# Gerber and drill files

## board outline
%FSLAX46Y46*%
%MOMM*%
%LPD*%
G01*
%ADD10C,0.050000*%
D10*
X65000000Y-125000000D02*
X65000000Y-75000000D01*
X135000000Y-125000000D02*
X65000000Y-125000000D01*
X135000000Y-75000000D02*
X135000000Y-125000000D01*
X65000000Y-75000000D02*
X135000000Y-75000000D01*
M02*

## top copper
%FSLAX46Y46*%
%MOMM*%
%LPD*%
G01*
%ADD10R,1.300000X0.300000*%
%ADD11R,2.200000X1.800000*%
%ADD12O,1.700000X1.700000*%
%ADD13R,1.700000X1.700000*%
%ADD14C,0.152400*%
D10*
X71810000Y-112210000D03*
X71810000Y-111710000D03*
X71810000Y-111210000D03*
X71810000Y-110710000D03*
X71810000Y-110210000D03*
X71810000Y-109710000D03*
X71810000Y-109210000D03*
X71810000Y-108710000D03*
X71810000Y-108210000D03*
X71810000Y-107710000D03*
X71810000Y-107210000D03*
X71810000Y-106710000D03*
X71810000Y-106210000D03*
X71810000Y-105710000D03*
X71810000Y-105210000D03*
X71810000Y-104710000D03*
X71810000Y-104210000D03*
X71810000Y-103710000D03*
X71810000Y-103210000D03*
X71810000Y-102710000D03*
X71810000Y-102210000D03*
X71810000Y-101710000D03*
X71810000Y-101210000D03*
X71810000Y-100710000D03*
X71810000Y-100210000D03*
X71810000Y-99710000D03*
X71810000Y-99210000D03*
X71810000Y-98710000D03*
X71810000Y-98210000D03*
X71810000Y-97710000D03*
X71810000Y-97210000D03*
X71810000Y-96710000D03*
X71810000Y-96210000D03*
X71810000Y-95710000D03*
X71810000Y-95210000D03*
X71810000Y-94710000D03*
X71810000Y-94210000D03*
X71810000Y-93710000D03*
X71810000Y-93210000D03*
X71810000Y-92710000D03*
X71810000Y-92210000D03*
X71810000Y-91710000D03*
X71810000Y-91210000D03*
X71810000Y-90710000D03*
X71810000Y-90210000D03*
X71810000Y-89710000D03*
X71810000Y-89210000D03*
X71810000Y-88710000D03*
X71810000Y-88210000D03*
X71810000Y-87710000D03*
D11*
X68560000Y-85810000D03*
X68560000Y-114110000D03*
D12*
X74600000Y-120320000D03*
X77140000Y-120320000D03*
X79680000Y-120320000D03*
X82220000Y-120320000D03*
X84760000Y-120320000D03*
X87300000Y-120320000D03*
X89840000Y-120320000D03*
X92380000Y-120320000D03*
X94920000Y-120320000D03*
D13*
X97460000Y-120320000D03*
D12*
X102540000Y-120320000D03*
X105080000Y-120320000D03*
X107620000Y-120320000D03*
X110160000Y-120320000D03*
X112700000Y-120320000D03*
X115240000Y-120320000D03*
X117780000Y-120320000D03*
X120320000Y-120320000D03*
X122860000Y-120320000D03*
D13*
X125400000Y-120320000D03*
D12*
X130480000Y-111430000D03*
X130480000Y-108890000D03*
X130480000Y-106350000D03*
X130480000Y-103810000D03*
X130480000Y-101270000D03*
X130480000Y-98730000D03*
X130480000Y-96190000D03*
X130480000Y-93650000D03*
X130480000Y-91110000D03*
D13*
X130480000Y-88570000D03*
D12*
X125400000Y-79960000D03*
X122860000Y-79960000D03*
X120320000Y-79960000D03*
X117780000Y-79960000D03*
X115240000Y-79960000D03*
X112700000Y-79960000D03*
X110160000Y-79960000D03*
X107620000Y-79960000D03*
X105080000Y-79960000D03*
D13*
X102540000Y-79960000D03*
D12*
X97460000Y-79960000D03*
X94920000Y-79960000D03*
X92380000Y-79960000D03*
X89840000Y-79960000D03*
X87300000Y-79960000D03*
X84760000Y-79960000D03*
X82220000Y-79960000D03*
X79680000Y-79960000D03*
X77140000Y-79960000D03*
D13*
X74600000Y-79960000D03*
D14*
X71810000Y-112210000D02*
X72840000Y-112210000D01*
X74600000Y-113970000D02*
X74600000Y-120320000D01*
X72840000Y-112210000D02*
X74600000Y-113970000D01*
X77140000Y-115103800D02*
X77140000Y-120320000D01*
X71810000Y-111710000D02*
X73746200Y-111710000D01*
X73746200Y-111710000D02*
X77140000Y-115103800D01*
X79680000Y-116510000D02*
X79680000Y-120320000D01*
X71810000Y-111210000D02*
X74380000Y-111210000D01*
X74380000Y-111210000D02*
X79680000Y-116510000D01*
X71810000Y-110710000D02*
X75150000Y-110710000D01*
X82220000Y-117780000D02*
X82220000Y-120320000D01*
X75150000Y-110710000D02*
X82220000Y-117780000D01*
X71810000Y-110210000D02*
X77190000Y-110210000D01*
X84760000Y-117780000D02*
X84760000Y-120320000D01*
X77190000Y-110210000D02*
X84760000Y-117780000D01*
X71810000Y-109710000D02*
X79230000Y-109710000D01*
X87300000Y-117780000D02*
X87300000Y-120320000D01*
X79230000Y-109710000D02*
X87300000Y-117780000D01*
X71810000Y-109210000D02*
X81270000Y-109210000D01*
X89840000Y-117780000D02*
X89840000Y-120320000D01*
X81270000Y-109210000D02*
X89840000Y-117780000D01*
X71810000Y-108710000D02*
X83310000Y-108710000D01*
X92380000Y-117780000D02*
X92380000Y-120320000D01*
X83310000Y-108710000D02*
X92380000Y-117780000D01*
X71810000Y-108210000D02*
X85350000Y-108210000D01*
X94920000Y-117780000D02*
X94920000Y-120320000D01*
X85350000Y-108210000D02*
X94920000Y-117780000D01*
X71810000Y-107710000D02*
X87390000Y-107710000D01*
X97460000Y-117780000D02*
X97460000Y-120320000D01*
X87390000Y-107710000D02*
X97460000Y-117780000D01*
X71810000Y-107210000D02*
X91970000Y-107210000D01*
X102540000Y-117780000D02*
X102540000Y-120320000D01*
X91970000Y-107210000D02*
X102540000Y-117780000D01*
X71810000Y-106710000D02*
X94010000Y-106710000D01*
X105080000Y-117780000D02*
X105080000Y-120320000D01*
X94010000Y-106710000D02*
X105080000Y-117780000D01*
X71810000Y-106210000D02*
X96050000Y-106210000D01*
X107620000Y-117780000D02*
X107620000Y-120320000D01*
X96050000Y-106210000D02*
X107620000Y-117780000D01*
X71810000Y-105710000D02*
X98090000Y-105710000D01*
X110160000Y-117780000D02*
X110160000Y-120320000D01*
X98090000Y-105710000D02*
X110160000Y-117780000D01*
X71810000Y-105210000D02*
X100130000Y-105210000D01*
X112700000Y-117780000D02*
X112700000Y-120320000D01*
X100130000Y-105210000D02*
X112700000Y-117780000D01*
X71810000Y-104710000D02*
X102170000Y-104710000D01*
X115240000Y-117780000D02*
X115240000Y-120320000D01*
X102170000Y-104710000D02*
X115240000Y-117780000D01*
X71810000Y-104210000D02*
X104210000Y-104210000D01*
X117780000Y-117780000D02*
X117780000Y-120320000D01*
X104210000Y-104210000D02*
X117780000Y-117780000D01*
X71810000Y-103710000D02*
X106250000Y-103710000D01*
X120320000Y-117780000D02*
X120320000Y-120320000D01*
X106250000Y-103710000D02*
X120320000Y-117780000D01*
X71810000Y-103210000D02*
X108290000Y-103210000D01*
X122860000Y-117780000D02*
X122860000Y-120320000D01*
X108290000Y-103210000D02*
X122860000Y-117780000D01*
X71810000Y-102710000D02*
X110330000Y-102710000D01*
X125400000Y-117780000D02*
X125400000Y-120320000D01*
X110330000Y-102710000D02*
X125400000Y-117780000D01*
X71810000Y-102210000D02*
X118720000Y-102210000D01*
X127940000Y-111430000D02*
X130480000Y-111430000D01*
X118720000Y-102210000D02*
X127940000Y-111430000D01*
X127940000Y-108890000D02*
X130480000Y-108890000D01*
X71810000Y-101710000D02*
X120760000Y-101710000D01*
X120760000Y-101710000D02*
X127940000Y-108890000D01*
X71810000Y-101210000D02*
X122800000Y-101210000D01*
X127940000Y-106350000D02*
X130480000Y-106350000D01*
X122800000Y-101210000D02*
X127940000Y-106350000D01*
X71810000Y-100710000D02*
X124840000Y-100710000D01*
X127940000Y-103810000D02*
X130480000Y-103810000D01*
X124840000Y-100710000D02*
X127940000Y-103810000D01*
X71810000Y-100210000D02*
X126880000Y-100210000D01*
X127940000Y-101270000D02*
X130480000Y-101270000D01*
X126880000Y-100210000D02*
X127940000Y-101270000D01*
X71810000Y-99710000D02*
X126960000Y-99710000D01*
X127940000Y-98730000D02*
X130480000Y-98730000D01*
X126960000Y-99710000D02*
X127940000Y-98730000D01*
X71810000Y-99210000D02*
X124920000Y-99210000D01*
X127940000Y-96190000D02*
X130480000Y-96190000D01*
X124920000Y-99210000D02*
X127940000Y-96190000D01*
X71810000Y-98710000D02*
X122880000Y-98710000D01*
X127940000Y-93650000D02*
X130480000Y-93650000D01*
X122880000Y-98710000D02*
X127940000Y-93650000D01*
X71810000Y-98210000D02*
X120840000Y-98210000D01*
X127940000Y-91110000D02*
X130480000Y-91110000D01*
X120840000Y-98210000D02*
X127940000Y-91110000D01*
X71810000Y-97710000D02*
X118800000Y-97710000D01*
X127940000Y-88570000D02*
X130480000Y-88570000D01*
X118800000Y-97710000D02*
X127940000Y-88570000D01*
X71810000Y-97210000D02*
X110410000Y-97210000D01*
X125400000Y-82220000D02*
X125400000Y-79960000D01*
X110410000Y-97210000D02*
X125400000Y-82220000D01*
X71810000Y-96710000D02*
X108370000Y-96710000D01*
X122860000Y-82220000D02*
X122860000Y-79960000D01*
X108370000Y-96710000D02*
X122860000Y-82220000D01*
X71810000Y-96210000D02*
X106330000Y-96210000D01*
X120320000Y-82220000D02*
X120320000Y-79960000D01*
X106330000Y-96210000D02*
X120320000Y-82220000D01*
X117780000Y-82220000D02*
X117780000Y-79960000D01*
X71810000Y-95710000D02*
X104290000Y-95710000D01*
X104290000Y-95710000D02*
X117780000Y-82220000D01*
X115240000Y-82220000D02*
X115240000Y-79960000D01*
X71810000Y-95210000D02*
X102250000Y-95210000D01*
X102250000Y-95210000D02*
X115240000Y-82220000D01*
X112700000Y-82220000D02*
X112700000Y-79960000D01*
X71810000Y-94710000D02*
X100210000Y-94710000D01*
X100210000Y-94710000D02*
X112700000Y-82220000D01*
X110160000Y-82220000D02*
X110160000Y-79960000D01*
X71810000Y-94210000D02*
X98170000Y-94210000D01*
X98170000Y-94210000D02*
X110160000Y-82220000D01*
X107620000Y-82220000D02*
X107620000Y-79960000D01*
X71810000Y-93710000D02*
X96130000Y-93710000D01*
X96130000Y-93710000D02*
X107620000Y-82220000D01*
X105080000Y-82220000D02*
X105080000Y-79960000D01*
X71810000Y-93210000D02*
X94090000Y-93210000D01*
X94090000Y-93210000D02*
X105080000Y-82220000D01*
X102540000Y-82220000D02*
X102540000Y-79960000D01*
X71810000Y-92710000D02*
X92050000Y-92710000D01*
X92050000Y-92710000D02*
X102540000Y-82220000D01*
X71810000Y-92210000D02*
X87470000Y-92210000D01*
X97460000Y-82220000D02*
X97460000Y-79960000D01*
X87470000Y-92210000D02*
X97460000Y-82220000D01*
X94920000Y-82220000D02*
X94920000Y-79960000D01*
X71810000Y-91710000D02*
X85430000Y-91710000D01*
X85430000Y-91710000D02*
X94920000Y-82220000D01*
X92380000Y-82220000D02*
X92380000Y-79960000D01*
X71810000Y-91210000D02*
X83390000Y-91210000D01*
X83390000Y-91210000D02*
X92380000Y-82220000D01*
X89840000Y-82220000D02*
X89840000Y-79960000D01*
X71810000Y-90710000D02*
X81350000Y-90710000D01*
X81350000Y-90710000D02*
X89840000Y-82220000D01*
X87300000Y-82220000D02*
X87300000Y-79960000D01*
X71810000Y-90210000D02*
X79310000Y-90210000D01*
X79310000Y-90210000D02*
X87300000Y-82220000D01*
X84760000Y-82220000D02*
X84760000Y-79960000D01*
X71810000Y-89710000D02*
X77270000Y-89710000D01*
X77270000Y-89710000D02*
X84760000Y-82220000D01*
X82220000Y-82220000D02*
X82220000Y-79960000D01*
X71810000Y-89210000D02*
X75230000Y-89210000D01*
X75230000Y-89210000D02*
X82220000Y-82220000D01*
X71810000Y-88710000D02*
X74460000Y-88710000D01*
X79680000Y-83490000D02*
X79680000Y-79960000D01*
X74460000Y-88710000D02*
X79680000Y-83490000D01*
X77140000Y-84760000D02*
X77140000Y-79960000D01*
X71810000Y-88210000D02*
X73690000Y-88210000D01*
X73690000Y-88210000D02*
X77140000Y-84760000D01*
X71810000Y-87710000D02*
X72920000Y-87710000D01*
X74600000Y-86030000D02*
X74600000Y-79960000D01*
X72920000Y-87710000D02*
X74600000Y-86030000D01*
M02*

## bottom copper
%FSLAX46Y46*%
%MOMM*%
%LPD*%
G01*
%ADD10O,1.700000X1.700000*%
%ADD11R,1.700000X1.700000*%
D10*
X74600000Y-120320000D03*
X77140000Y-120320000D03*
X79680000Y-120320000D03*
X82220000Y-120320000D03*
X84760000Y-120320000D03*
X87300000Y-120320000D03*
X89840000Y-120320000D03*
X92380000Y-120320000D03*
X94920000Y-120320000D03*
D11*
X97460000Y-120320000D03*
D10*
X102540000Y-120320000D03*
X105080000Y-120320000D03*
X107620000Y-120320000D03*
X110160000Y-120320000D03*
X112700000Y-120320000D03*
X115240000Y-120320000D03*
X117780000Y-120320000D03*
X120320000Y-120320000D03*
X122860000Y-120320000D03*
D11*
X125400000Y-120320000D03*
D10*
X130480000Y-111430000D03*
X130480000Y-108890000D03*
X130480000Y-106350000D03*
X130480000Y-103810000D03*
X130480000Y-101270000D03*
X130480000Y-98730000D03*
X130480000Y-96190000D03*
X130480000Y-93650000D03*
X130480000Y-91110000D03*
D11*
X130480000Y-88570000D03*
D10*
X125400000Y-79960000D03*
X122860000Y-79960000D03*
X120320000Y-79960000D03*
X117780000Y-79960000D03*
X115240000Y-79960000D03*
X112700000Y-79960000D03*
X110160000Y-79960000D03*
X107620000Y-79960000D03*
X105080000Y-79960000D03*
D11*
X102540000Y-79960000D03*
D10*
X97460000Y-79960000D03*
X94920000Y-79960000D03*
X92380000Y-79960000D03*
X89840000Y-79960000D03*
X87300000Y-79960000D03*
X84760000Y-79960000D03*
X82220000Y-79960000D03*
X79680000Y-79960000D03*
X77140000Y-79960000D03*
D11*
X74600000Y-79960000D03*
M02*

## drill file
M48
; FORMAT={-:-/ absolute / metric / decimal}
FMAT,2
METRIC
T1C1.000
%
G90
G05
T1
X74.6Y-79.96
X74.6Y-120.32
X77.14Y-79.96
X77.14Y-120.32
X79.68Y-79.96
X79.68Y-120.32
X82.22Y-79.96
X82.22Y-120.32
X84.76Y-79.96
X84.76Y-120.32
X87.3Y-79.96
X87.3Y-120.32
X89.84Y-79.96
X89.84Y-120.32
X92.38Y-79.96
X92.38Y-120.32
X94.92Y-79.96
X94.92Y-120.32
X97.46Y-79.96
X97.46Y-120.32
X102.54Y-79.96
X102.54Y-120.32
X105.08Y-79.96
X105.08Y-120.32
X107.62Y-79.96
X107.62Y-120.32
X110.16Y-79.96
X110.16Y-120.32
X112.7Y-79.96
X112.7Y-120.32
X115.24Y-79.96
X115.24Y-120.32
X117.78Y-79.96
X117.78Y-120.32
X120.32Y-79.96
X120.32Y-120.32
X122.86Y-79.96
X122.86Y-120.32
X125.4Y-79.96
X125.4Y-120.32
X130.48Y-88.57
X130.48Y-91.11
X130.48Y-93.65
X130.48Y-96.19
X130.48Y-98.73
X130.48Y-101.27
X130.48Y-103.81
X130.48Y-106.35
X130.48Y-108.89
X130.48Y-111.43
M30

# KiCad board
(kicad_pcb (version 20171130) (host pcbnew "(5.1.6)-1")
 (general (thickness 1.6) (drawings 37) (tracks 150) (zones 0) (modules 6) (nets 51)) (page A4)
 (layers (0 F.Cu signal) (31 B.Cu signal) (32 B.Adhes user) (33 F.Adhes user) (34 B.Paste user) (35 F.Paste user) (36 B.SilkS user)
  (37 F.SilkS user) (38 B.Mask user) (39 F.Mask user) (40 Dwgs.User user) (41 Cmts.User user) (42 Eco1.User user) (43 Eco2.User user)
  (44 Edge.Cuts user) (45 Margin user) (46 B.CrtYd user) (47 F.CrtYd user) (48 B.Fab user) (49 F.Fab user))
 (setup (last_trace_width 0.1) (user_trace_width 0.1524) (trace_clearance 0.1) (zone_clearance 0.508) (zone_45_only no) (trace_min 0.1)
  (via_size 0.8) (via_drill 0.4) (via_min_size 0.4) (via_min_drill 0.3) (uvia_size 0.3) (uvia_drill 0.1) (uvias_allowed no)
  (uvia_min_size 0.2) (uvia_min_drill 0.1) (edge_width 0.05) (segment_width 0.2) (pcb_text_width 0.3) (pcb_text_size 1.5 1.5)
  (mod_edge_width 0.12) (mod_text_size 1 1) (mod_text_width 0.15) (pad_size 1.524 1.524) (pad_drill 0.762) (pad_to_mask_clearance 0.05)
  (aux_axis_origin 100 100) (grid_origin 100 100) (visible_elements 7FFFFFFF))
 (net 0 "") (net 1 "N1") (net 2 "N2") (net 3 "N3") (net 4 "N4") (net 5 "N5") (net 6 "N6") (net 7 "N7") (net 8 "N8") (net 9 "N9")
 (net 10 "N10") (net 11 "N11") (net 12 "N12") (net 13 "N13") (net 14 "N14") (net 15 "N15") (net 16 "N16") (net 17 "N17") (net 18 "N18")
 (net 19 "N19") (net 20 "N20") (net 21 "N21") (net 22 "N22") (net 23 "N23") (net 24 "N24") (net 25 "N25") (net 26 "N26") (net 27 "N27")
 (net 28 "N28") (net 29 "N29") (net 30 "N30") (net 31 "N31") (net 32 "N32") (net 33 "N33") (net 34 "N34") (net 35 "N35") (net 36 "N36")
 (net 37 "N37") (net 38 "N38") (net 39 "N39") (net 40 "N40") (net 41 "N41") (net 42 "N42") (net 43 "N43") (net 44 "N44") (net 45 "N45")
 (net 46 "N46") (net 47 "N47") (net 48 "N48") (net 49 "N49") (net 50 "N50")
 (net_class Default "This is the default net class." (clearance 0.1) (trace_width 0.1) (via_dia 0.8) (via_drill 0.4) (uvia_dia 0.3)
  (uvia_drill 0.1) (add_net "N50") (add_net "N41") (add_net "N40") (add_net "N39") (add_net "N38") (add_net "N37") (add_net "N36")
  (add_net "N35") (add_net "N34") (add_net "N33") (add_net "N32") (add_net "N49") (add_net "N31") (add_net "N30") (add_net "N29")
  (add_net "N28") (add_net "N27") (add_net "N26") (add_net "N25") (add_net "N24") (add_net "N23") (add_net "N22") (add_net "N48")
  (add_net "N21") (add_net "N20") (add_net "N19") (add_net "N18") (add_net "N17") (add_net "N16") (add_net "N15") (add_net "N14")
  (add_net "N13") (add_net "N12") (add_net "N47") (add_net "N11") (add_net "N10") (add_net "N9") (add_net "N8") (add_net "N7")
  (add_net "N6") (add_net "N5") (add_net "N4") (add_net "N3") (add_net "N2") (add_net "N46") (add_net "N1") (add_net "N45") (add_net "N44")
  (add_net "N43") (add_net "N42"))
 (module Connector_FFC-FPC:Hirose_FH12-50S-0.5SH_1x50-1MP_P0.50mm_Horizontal (layer F.Cu) (at 69.96 99.96 270)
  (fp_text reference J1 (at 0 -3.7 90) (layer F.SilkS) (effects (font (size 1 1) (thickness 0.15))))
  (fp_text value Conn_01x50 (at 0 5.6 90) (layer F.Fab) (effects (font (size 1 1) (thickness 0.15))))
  (pad 50 smd rect (at 12.25 -1.85 270) (size 0.3 1.3) (layers F.Cu F.Paste F.Mask) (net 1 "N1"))
  (pad 49 smd rect (at 11.75 -1.85 270) (size 0.3 1.3) (layers F.Cu F.Paste F.Mask) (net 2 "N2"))
  (pad 48 smd rect (at 11.25 -1.85 270) (size 0.3 1.3) (layers F.Cu F.Paste F.Mask) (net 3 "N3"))
  (pad 47 smd rect (at 10.75 -1.85 270) (size 0.3 1.3) (layers F.Cu F.Paste F.Mask) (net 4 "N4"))
  (pad 46 smd rect (at 10.25 -1.85 270) (size 0.3 1.3) (layers F.Cu F.Paste F.Mask) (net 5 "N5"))
  (pad 45 smd rect (at 9.75 -1.85 270) (size 0.3 1.3) (layers F.Cu F.Paste F.Mask) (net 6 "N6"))
  (pad 44 smd rect (at 9.25 -1.85 270) (size 0.3 1.3) (layers F.Cu F.Paste F.Mask) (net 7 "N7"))
  (pad 43 smd rect (at 8.75 -1.85 270) (size 0.3 1.3) (layers F.Cu F.Paste F.Mask) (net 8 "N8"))
  (pad 42 smd rect (at 8.25 -1.85 270) (size 0.3 1.3) (layers F.Cu F.Paste F.Mask) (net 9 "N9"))
  (pad 41 smd rect (at 7.75 -1.85 270) (size 0.3 1.3) (layers F.Cu F.Paste F.Mask) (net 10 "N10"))
  (pad 40 smd rect (at 7.25 -1.85 270) (size 0.3 1.3) (layers F.Cu F.Paste F.Mask) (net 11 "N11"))
  (pad 39 smd rect (at 6.75 -1.85 270) (size 0.3 1.3) (layers F.Cu F.Paste F.Mask) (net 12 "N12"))
  (pad 38 smd rect (at 6.25 -1.85 270) (size 0.3 1.3) (layers F.Cu F.Paste F.Mask) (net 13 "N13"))
  (pad 37 smd rect (at 5.75 -1.85 270) (size 0.3 1.3) (layers F.Cu F.Paste F.Mask) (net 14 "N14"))
  (pad 36 smd rect (at 5.25 -1.85 270) (size 0.3 1.3) (layers F.Cu F.Paste F.Mask) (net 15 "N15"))
  (pad 35 smd rect (at 4.75 -1.85 270) (size 0.3 1.3) (layers F.Cu F.Paste F.Mask) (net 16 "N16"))
  (pad 34 smd rect (at 4.25 -1.85 270) (size 0.3 1.3) (layers F.Cu F.Paste F.Mask) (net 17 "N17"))
  (pad 33 smd rect (at 3.75 -1.85 270) (size 0.3 1.3) (layers F.Cu F.Paste F.Mask) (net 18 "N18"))
  (pad 32 smd rect (at 3.25 -1.85 270) (size 0.3 1.3) (layers F.Cu F.Paste F.Mask) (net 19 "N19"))
  (pad 31 smd rect (at 2.75 -1.85 270) (size 0.3 1.3) (layers F.Cu F.Paste F.Mask) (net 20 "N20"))
  (pad 30 smd rect (at 2.25 -1.85 270) (size 0.3 1.3) (layers F.Cu F.Paste F.Mask) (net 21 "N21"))
  (pad 29 smd rect (at 1.75 -1.85 270) (size 0.3 1.3) (layers F.Cu F.Paste F.Mask) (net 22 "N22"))
  (pad 28 smd rect (at 1.25 -1.85 270) (size 0.3 1.3) (layers F.Cu F.Paste F.Mask) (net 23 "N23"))
  (pad 27 smd rect (at 0.75 -1.85 270) (size 0.3 1.3) (layers F.Cu F.Paste F.Mask) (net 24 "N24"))
  (pad 26 smd rect (at 0.25 -1.85 270) (size 0.3 1.3) (layers F.Cu F.Paste F.Mask) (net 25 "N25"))
  (pad 25 smd rect (at -0.25 -1.85 270) (size 0.3 1.3) (layers F.Cu F.Paste F.Mask) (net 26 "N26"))
  (pad 24 smd rect (at -0.75 -1.85 270) (size 0.3 1.3) (layers F.Cu F.Paste F.Mask) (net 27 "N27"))
  (pad 23 smd rect (at -1.25 -1.85 270) (size 0.3 1.3) (layers F.Cu F.Paste F.Mask) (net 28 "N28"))
  (pad 22 smd rect (at -1.75 -1.85 270) (size 0.3 1.3) (layers F.Cu F.Paste F.Mask) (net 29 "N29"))
  (pad 21 smd rect (at -2.25 -1.85 270) (size 0.3 1.3) (layers F.Cu F.Paste F.Mask) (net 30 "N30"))
  (pad 20 smd rect (at -2.75 -1.85 270) (size 0.3 1.3) (layers F.Cu F.Paste F.Mask) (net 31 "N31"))
  (pad 19 smd rect (at -3.25 -1.85 270) (size 0.3 1.3) (layers F.Cu F.Paste F.Mask) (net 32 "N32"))
  (pad 18 smd rect (at -3.75 -1.85 270) (size 0.3 1.3) (layers F.Cu F.Paste F.Mask) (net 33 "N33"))
  (pad 17 smd rect (at -4.25 -1.85 270) (size 0.3 1.3) (layers F.Cu F.Paste F.Mask) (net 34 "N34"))
  (pad 16 smd rect (at -4.75 -1.85 270) (size 0.3 1.3) (layers F.Cu F.Paste F.Mask) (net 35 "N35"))
  (pad 15 smd rect (at -5.25 -1.85 270) (size 0.3 1.3) (layers F.Cu F.Paste F.Mask) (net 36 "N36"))
  (pad 14 smd rect (at -5.75 -1.85 270) (size 0.3 1.3) (layers F.Cu F.Paste F.Mask) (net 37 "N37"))
  (pad 13 smd rect (at -6.25 -1.85 270) (size 0.3 1.3) (layers F.Cu F.Paste F.Mask) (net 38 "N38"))
  (pad 12 smd rect (at -6.75 -1.85 270) (size 0.3 1.3) (layers F.Cu F.Paste F.Mask) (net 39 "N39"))
  (pad 11 smd rect (at -7.25 -1.85 270) (size 0.3 1.3) (layers F.Cu F.Paste F.Mask) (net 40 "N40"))
  (pad 10 smd rect (at -7.75 -1.85 270) (size 0.3 1.3) (layers F.Cu F.Paste F.Mask) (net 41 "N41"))
  (pad 9 smd rect (at -8.25 -1.85 270) (size 0.3 1.3) (layers F.Cu F.Paste F.Mask) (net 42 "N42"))
  (pad 8 smd rect (at -8.75 -1.85 270) (size 0.3 1.3) (layers F.Cu F.Paste F.Mask) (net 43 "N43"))
  (pad 7 smd rect (at -9.25 -1.85 270) (size 0.3 1.3) (layers F.Cu F.Paste F.Mask) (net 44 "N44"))
  (pad 6 smd rect (at -9.75 -1.85 270) (size 0.3 1.3) (layers F.Cu F.Paste F.Mask) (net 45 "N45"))
  (pad 5 smd rect (at -10.25 -1.85 270) (size 0.3 1.3) (layers F.Cu F.Paste F.Mask) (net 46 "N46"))
  (pad 4 smd rect (at -10.75 -1.85 270) (size 0.3 1.3) (layers F.Cu F.Paste F.Mask) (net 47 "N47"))
  (pad 3 smd rect (at -11.25 -1.85 270) (size 0.3 1.3) (layers F.Cu F.Paste F.Mask) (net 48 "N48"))
  (pad 2 smd rect (at -11.75 -1.85 270) (size 0.3 1.3) (layers F.Cu F.Paste F.Mask) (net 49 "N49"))
  (pad 1 smd rect (at -12.25 -1.85 270) (size 0.3 1.3) (layers F.Cu F.Paste F.Mask) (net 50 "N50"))
  (pad MP smd rect (at -14.15 1.4 270) (size 1.8 2.2) (layers F.Cu F.Paste F.Mask))
  (pad MP smd rect (at 14.15 1.4 270) (size 1.8 2.2) (layers F.Cu F.Paste F.Mask)))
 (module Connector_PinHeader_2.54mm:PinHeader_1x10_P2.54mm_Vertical (layer F.Cu) (at 97.46 120.32 270)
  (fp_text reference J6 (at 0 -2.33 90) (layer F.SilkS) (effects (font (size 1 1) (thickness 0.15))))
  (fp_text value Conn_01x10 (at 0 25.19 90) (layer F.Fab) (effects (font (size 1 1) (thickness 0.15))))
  (pad 10 thru_hole oval (at 0 22.86 270) (size 1.7 1.7) (drill 1) (layers *.Cu *.Mask) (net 1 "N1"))
  (pad 9 thru_hole oval (at 0 20.32 270) (size 1.7 1.7) (drill 1) (layers *.Cu *.Mask) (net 2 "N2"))
  (pad 8 thru_hole oval (at 0 17.78 270) (size 1.7 1.7) (drill 1) (layers *.Cu *.Mask) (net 3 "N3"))
  (pad 7 thru_hole oval (at 0 15.24 270) (size 1.7 1.7) (drill 1) (layers *.Cu *.Mask) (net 4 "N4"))
  (pad 6 thru_hole oval (at 0 12.7 270) (size 1.7 1.7) (drill 1) (layers *.Cu *.Mask) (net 5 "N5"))
  (pad 5 thru_hole oval (at 0 10.16 270) (size 1.7 1.7) (drill 1) (layers *.Cu *.Mask) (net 6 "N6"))
  (pad 4 thru_hole oval (at 0 7.62 270) (size 1.7 1.7) (drill 1) (layers *.Cu *.Mask) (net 7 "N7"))
  (pad 3 thru_hole oval (at 0 5.08 270) (size 1.7 1.7) (drill 1) (layers *.Cu *.Mask) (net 8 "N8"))
  (pad 2 thru_hole oval (at 0 2.54 270) (size 1.7 1.7) (drill 1) (layers *.Cu *.Mask) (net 9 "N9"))
  (pad 1 thru_hole rect (at 0 0 270) (size 1.7 1.7) (drill 1) (layers *.Cu *.Mask) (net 10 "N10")))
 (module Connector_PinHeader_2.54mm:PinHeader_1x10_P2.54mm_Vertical (layer F.Cu) (at 125.4 120.32 270)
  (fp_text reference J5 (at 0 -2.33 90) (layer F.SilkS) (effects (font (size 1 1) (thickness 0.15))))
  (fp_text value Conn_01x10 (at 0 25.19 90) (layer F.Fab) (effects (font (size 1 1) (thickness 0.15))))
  (pad 10 thru_hole oval (at 0 22.86 270) (size 1.7 1.7) (drill 1) (layers *.Cu *.Mask) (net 11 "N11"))
  (pad 9 thru_hole oval (at 0 20.32 270) (size 1.7 1.7) (drill 1) (layers *.Cu *.Mask) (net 12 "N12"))
  (pad 8 thru_hole oval (at 0 17.78 270) (size 1.7 1.7) (drill 1) (layers *.Cu *.Mask) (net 13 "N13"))
  (pad 7 thru_hole oval (at 0 15.24 270) (size 1.7 1.7) (drill 1) (layers *.Cu *.Mask) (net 14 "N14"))
  (pad 6 thru_hole oval (at 0 12.7 270) (size 1.7 1.7) (drill 1) (layers *.Cu *.Mask) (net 15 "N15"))
  (pad 5 thru_hole oval (at 0 10.16 270) (size 1.7 1.7) (drill 1) (layers *.Cu *.Mask) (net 16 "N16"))
  (pad 4 thru_hole oval (at 0 7.62 270) (size 1.7 1.7) (drill 1) (layers *.Cu *.Mask) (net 17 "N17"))
  (pad 3 thru_hole oval (at 0 5.08 270) (size 1.7 1.7) (drill 1) (layers *.Cu *.Mask) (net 18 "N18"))
  (pad 2 thru_hole oval (at 0 2.54 270) (size 1.7 1.7) (drill 1) (layers *.Cu *.Mask) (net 19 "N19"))
  (pad 1 thru_hole rect (at 0 0 270) (size 1.7 1.7) (drill 1) (layers *.Cu *.Mask) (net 20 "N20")))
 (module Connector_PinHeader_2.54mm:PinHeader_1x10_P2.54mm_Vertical (layer F.Cu) (at 130.48 88.57)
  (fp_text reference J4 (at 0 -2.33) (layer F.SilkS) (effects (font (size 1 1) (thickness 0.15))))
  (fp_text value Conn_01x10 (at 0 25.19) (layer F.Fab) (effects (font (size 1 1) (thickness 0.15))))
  (pad 10 thru_hole oval (at 0 22.86) (size 1.7 1.7) (drill 1) (layers *.Cu *.Mask) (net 21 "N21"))
  (pad 9 thru_hole oval (at 0 20.32) (size 1.7 1.7) (drill 1) (layers *.Cu *.Mask) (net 22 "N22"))
  (pad 8 thru_hole oval (at 0 17.78) (size 1.7 1.7) (drill 1) (layers *.Cu *.Mask) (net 23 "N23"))
  (pad 7 thru_hole oval (at 0 15.24) (size 1.7 1.7) (drill 1) (layers *.Cu *.Mask) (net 24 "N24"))
  (pad 6 thru_hole oval (at 0 12.7) (size 1.7 1.7) (drill 1) (layers *.Cu *.Mask) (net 25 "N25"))
  (pad 5 thru_hole oval (at 0 10.16) (size 1.7 1.7) (drill 1) (layers *.Cu *.Mask) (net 26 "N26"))
  (pad 4 thru_hole oval (at 0 7.62) (size 1.7 1.7) (drill 1) (layers *.Cu *.Mask) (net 27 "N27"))
  (pad 3 thru_hole oval (at 0 5.08) (size 1.7 1.7) (drill 1) (layers *.Cu *.Mask) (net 28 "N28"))
  (pad 2 thru_hole oval (at 0 2.54) (size 1.7 1.7) (drill 1) (layers *.Cu *.Mask) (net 29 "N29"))
  (pad 1 thru_hole rect (at 0 0) (size 1.7 1.7) (drill 1) (layers *.Cu *.Mask) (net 30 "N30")))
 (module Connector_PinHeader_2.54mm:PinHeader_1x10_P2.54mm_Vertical (layer F.Cu) (at 102.54 79.96 90)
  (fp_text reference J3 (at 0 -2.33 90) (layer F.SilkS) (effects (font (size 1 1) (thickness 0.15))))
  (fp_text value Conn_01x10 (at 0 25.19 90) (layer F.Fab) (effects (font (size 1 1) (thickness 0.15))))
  (pad 10 thru_hole oval (at 0 22.86 90) (size 1.7 1.7) (drill 1) (layers *.Cu *.Mask) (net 31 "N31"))
  (pad 9 thru_hole oval (at 0 20.32 90) (size 1.7 1.7) (drill 1) (layers *.Cu *.Mask) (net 32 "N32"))
  (pad 8 thru_hole oval (at 0 17.78 90) (size 1.7 1.7) (drill 1) (layers *.Cu *.Mask) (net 33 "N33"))
  (pad 7 thru_hole oval (at 0 15.24 90) (size 1.7 1.7) (drill 1) (layers *.Cu *.Mask) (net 34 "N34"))
  (pad 6 thru_hole oval (at 0 12.7 90) (size 1.7 1.7) (drill 1) (layers *.Cu *.Mask) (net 35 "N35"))
  (pad 5 thru_hole oval (at 0 10.16 90) (size 1.7 1.7) (drill 1) (layers *.Cu *.Mask) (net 36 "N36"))
  (pad 4 thru_hole oval (at 0 7.62 90) (size 1.7 1.7) (drill 1) (layers *.Cu *.Mask) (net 37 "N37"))
  (pad 3 thru_hole oval (at 0 5.08 90) (size 1.7 1.7) (drill 1) (layers *.Cu *.Mask) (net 38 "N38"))
  (pad 2 thru_hole oval (at 0 2.54 90) (size 1.7 1.7) (drill 1) (layers *.Cu *.Mask) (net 39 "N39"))
  (pad 1 thru_hole rect (at 0 0 90) (size 1.7 1.7) (drill 1) (layers *.Cu *.Mask) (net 40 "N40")))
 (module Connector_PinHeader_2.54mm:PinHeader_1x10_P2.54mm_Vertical (layer F.Cu) (at 74.6 79.96 90)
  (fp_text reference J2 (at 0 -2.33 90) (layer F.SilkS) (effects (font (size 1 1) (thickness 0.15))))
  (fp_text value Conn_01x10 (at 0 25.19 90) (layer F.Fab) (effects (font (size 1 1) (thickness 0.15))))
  (pad 10 thru_hole oval (at 0 22.86 90) (size 1.7 1.7) (drill 1) (layers *.Cu *.Mask) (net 41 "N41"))
  (pad 9 thru_hole oval (at 0 20.32 90) (size 1.7 1.7) (drill 1) (layers *.Cu *.Mask) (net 42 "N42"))
  (pad 8 thru_hole oval (at 0 17.78 90) (size 1.7 1.7) (drill 1) (layers *.Cu *.Mask) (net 43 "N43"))
  (pad 7 thru_hole oval (at 0 15.24 90) (size 1.7 1.7) (drill 1) (layers *.Cu *.Mask) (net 44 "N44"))
  (pad 6 thru_hole oval (at 0 12.7 90) (size 1.7 1.7) (drill 1) (layers *.Cu *.Mask) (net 45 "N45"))
  (pad 5 thru_hole oval (at 0 10.16 90) (size 1.7 1.7) (drill 1) (layers *.Cu *.Mask) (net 46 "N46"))
  (pad 4 thru_hole oval (at 0 7.62 90) (size 1.7 1.7) (drill 1) (layers *.Cu *.Mask) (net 47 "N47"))
  (pad 3 thru_hole oval (at 0 5.08 90) (size 1.7 1.7) (drill 1) (layers *.Cu *.Mask) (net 48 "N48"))
  (pad 2 thru_hole oval (at 0 2.54 90) (size 1.7 1.7) (drill 1) (layers *.Cu *.Mask) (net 49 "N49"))
  (pad 1 thru_hole rect (at 0 0 90) (size 1.7 1.7) (drill 1) (layers *.Cu *.Mask) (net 50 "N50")))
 (gr_line (start 65 125) (end 65 75) (layer Edge.Cuts) (width 0.05))
 (gr_line (start 135 125) (end 65 125) (layer Edge.Cuts) (width 0.05))
 (gr_line (start 135 75) (end 135 125) (layer Edge.Cuts) (width 0.05))
 (gr_line (start 65 75) (end 135 75) (layer Edge.Cuts) (width 0.05))
 (segment (start 71.81 112.21) (end 72.84 112.21) (width 0.1524) (layer F.Cu) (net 1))
 (segment (start 74.6 113.97) (end 74.6 120.32) (width 0.1524) (layer F.Cu) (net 1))
 (segment (start 72.84 112.21) (end 74.6 113.97) (width 0.1524) (layer F.Cu) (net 1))
 (segment (start 77.14 115.1038) (end 77.14 120.32) (width 0.1524) (layer F.Cu) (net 2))
 (segment (start 71.81 111.71) (end 73.7462 111.71) (width 0.1524) (layer F.Cu) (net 2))
 (segment (start 73.7462 111.71) (end 77.14 115.1038) (width 0.1524) (layer F.Cu) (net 2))
 (segment (start 79.68 116.51) (end 79.68 120.32) (width 0.1524) (layer F.Cu) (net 3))
 (segment (start 71.81 111.21) (end 74.38 111.21) (width 0.1524) (layer F.Cu) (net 3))
 (segment (start 74.38 111.21) (end 79.68 116.51) (width 0.1524) (layer F.Cu) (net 3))
 (segment (start 71.81 110.71) (end 75.15 110.71) (width 0.1524) (layer F.Cu) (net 4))
 (segment (start 82.22 117.78) (end 82.22 120.32) (width 0.1524) (layer F.Cu) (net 4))
 (segment (start 75.15 110.71) (end 82.22 117.78) (width 0.1524) (layer F.Cu) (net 4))
 (segment (start 71.81 110.21) (end 77.19 110.21) (width 0.1524) (layer F.Cu) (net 5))
 (segment (start 84.76 117.78) (end 84.76 120.32) (width 0.1524) (layer F.Cu) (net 5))
 (segment (start 77.19 110.21) (end 84.76 117.78) (width 0.1524) (layer F.Cu) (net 5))
 (segment (start 71.81 109.71) (end 79.23 109.71) (width 0.1524) (layer F.Cu) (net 6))
 (segment (start 87.3 117.78) (end 87.3 120.32) (width 0.1524) (layer F.Cu) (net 6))
 (segment (start 79.23 109.71) (end 87.3 117.78) (width 0.1524) (layer F.Cu) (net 6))
 (segment (start 71.81 109.21) (end 81.27 109.21) (width 0.1524) (layer F.Cu) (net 7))
 (segment (start 89.84 117.78) (end 89.84 120.32) (width 0.1524) (layer F.Cu) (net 7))
 (segment (start 81.27 109.21) (end 89.84 117.78) (width 0.1524) (layer F.Cu) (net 7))
 (segment (start 71.81 108.71) (end 83.31 108.71) (width 0.1524) (layer F.Cu) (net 8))
 (segment (start 92.38 117.78) (end 92.38 120.32) (width 0.1524) (layer F.Cu) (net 8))
 (segment (start 83.31 108.71) (end 92.38 117.78) (width 0.1524) (layer F.Cu) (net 8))
 (segment (start 71.81 108.21) (end 85.35 108.21) (width 0.1524) (layer F.Cu) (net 9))
 (segment (start 94.92 117.78) (end 94.92 120.32) (width 0.1524) (layer F.Cu) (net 9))
 (segment (start 85.35 108.21) (end 94.92 117.78) (width 0.1524) (layer F.Cu) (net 9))
 (segment (start 71.81 107.71) (end 87.39 107.71) (width 0.1524) (layer F.Cu) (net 10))
 (segment (start 97.46 117.78) (end 97.46 120.32) (width 0.1524) (layer F.Cu) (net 10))
 (segment (start 87.39 107.71) (end 97.46 117.78) (width 0.1524) (layer F.Cu) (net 10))
 (segment (start 71.81 107.21) (end 91.97 107.21) (width 0.1524) (layer F.Cu) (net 11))
 (segment (start 102.54 117.78) (end 102.54 120.32) (width 0.1524) (layer F.Cu) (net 11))
 (segment (start 91.97 107.21) (end 102.54 117.78) (width 0.1524) (layer F.Cu) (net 11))
 (segment (start 71.81 106.71) (end 94.01 106.71) (width 0.1524) (layer F.Cu) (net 12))
 (segment (start 105.08 117.78) (end 105.08 120.32) (width 0.1524) (layer F.Cu) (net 12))
 (segment (start 94.01 106.71) (end 105.08 117.78) (width 0.1524) (layer F.Cu) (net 12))
 (segment (start 71.81 106.21) (end 96.05 106.21) (width 0.1524) (layer F.Cu) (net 13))
 (segment (start 107.62 117.78) (end 107.62 120.32) (width 0.1524) (layer F.Cu) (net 13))
 (segment (start 96.05 106.21) (end 107.62 117.78) (width 0.1524) (layer F.Cu) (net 13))
 (segment (start 71.81 105.71) (end 98.09 105.71) (width 0.1524) (layer F.Cu) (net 14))
 (segment (start 110.16 117.78) (end 110.16 120.32) (width 0.1524) (layer F.Cu) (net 14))
 (segment (start 98.09 105.71) (end 110.16 117.78) (width 0.1524) (layer F.Cu) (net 14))
 (segment (start 71.81 105.21) (end 100.13 105.21) (width 0.1524) (layer F.Cu) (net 15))
 (segment (start 112.7 117.78) (end 112.7 120.32) (width 0.1524) (layer F.Cu) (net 15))
 (segment (start 100.13 105.21) (end 112.7 117.78) (width 0.1524) (layer F.Cu) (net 15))
 (segment (start 71.81 104.71) (end 102.17 104.71) (width 0.1524) (layer F.Cu) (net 16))
 (segment (start 115.24 117.78) (end 115.24 120.32) (width 0.1524) (layer F.Cu) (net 16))
 (segment (start 102.17 104.71) (end 115.24 117.78) (width 0.1524) (layer F.Cu) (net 16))
 (segment (start 71.81 104.21) (end 104.21 104.21) (width 0.1524) (layer F.Cu) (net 17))
 (segment (start 117.78 117.78) (end 117.78 120.32) (width 0.1524) (layer F.Cu) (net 17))
 (segment (start 104.21 104.21) (end 117.78 117.78) (width 0.1524) (layer F.Cu) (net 17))
 (segment (start 71.81 103.71) (end 106.25 103.71) (width 0.1524) (layer F.Cu) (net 18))
 (segment (start 120.32 117.78) (end 120.32 120.32) (width 0.1524) (layer F.Cu) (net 18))
 (segment (start 106.25 103.71) (end 120.32 117.78) (width 0.1524) (layer F.Cu) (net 18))
 (segment (start 71.81 103.21) (end 108.29 103.21) (width 0.1524) (layer F.Cu) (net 19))
 (segment (start 122.86 117.78) (end 122.86 120.32) (width 0.1524) (layer F.Cu) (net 19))
 (segment (start 108.29 103.21) (end 122.86 117.78) (width 0.1524) (layer F.Cu) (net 19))
 (segment (start 71.81 102.71) (end 110.33 102.71) (width 0.1524) (layer F.Cu) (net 20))
 (segment (start 125.4 117.78) (end 125.4 120.32) (width 0.1524) (layer F.Cu) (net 20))
 (segment (start 110.33 102.71) (end 125.4 117.78) (width 0.1524) (layer F.Cu) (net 20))
 (segment (start 71.81 102.21) (end 118.72 102.21) (width 0.1524) (layer F.Cu) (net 21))
 (segment (start 127.94 111.43) (end 130.48 111.43) (width 0.1524) (layer F.Cu) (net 21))
 (segment (start 118.72 102.21) (end 127.94 111.43) (width 0.1524) (layer F.Cu) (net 21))
 (segment (start 127.94 108.89) (end 130.48 108.89) (width 0.1524) (layer F.Cu) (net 22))
 (segment (start 71.81 101.71) (end 120.76 101.71) (width 0.1524) (layer F.Cu) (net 22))
 (segment (start 120.76 101.71) (end 127.94 108.89) (width 0.1524) (layer F.Cu) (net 22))
 (segment (start 71.81 101.21) (end 122.8 101.21) (width 0.1524) (layer F.Cu) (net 23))
 (segment (start 127.94 106.35) (end 130.48 106.35) (width 0.1524) (layer F.Cu) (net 23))
 (segment (start 122.8 101.21) (end 127.94 106.35) (width 0.1524) (layer F.Cu) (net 23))
 (segment (start 71.81 100.71) (end 124.84 100.71) (width 0.1524) (layer F.Cu) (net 24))
 (segment (start 127.94 103.81) (end 130.48 103.81) (width 0.1524) (layer F.Cu) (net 24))
 (segment (start 124.84 100.71) (end 127.94 103.81) (width 0.1524) (layer F.Cu) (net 24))
 (segment (start 71.81 100.21) (end 126.88 100.21) (width 0.1524) (layer F.Cu) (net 25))
 (segment (start 127.94 101.27) (end 130.48 101.27) (width 0.1524) (layer F.Cu) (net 25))
 (segment (start 126.88 100.21) (end 127.94 101.27) (width 0.1524) (layer F.Cu) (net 25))
 (segment (start 71.81 99.71) (end 126.96 99.71) (width 0.1524) (layer F.Cu) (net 26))
 (segment (start 127.94 98.73) (end 130.48 98.73) (width 0.1524) (layer F.Cu) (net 26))
 (segment (start 126.96 99.71) (end 127.94 98.73) (width 0.1524) (layer F.Cu) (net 26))
 (segment (start 71.81 99.21) (end 124.92 99.21) (width 0.1524) (layer F.Cu) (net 27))
 (segment (start 127.94 96.19) (end 130.48 96.19) (width 0.1524) (layer F.Cu) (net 27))
 (segment (start 124.92 99.21) (end 127.94 96.19) (width 0.1524) (layer F.Cu) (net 27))
 (segment (start 71.81 98.71) (end 122.88 98.71) (width 0.1524) (layer F.Cu) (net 28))
 (segment (start 127.94 93.65) (end 130.48 93.65) (width 0.1524) (layer F.Cu) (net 28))
 (segment (start 122.88 98.71) (end 127.94 93.65) (width 0.1524) (layer F.Cu) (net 28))
 (segment (start 71.81 98.21) (end 120.84 98.21) (width 0.1524) (layer F.Cu) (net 29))
 (segment (start 127.94 91.11) (end 130.48 91.11) (width 0.1524) (layer F.Cu) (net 29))
 (segment (start 120.84 98.21) (end 127.94 91.11) (width 0.1524) (layer F.Cu) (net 29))
 (segment (start 71.81 97.71) (end 118.8 97.71) (width 0.1524) (layer F.Cu) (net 30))
 (segment (start 127.94 88.57) (end 130.48 88.57) (width 0.1524) (layer F.Cu) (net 30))
 (segment (start 118.8 97.71) (end 127.94 88.57) (width 0.1524) (layer F.Cu) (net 30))
 (segment (start 71.81 97.21) (end 110.41 97.21) (width 0.1524) (layer F.Cu) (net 31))
 (segment (start 125.4 82.22) (end 125.4 79.96) (width 0.1524) (layer F.Cu) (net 31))
 (segment (start 110.41 97.21) (end 125.4 82.22) (width 0.1524) (layer F.Cu) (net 31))
 (segment (start 71.81 96.71) (end 108.37 96.71) (width 0.1524) (layer F.Cu) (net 32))
 (segment (start 122.86 82.22) (end 122.86 79.96) (width 0.1524) (layer F.Cu) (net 32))
 (segment (start 108.37 96.71) (end 122.86 82.22) (width 0.1524) (layer F.Cu) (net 32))
 (segment (start 71.81 96.21) (end 106.33 96.21) (width 0.1524) (layer F.Cu) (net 33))
 (segment (start 120.32 82.22) (end 120.32 79.96) (width 0.1524) (layer F.Cu) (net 33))
 (segment (start 106.33 96.21) (end 120.32 82.22) (width 0.1524) (layer F.Cu) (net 33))
 (segment (start 117.78 82.22) (end 117.78 79.96) (width 0.1524) (layer F.Cu) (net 34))
 (segment (start 71.81 95.71) (end 104.29 95.71) (width 0.1524) (layer F.Cu) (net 34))
 (segment (start 104.29 95.71) (end 117.78 82.22) (width 0.1524) (layer F.Cu) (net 34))
 (segment (start 115.24 82.22) (end 115.24 79.96) (width 0.1524) (layer F.Cu) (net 35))
 (segment (start 71.81 95.21) (end 102.25 95.21) (width 0.1524) (layer F.Cu) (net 35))
 (segment (start 102.25 95.21) (end 115.24 82.22) (width 0.1524) (layer F.Cu) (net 35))
 (segment (start 112.7 82.22) (end 112.7 79.96) (width 0.1524) (layer F.Cu) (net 36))
 (segment (start 71.81 94.71) (end 100.21 94.71) (width 0.1524) (layer F.Cu) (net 36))
 (segment (start 100.21 94.71) (end 112.7 82.22) (width 0.1524) (layer F.Cu) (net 36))
 (segment (start 110.16 82.22) (end 110.16 79.96) (width 0.1524) (layer F.Cu) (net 37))
 (segment (start 71.81 94.21) (end 98.17 94.21) (width 0.1524) (layer F.Cu) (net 37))
 (segment (start 98.17 94.21) (end 110.16 82.22) (width 0.1524) (layer F.Cu) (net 37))
 (segment (start 107.62 82.22) (end 107.62 79.96) (width 0.1524) (layer F.Cu) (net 38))
 (segment (start 71.81 93.71) (end 96.13 93.71) (width 0.1524) (layer F.Cu) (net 38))
 (segment (start 96.13 93.71) (end 107.62 82.22) (width 0.1524) (layer F.Cu) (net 38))
 (segment (start 105.08 82.22) (end 105.08 79.96) (width 0.1524) (layer F.Cu) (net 39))
 (segment (start 71.81 93.21) (end 94.09 93.21) (width 0.1524) (layer F.Cu) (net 39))
 (segment (start 94.09 93.21) (end 105.08 82.22) (width 0.1524) (layer F.Cu) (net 39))
 (segment (start 102.54 82.22) (end 102.54 79.96) (width 0.1524) (layer F.Cu) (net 40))
 (segment (start 71.81 92.71) (end 92.05 92.71) (width 0.1524) (layer F.Cu) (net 40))
 (segment (start 92.05 92.71) (end 102.54 82.22) (width 0.1524) (layer F.Cu) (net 40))
 (segment (start 71.81 92.21) (end 87.47 92.21) (width 0.1524) (layer F.Cu) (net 41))
 (segment (start 97.46 82.22) (end 97.46 79.96) (width 0.1524) (layer F.Cu) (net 41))
 (segment (start 87.47 92.21) (end 97.46 82.22) (width 0.1524) (layer F.Cu) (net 41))
 (segment (start 94.92 82.22) (end 94.92 79.96) (width 0.1524) (layer F.Cu) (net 42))
 (segment (start 71.81 91.71) (end 85.43 91.71) (width 0.1524) (layer F.Cu) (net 42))
 (segment (start 85.43 91.71) (end 94.92 82.22) (width 0.1524) (layer F.Cu) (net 42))
 (segment (start 92.38 82.22) (end 92.38 79.96) (width 0.1524) (layer F.Cu) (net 43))
 (segment (start 71.81 91.21) (end 83.39 91.21) (width 0.1524) (layer F.Cu) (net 43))
 (segment (start 83.39 91.21) (end 92.38 82.22) (width 0.1524) (layer F.Cu) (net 43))
 (segment (start 89.84 82.22) (end 89.84 79.96) (width 0.1524) (layer F.Cu) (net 44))
 (segment (start 71.81 90.71) (end 81.35 90.71) (width 0.1524) (layer F.Cu) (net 44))
 (segment (start 81.35 90.71) (end 89.84 82.22) (width 0.1524) (layer F.Cu) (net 44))
 (segment (start 87.3 82.22) (end 87.3 79.96) (width 0.1524) (layer F.Cu) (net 45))
 (segment (start 71.81 90.21) (end 79.31 90.21) (width 0.1524) (layer F.Cu) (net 45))
 (segment (start 79.31 90.21) (end 87.3 82.22) (width 0.1524) (layer F.Cu) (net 45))
 (segment (start 84.76 82.22) (end 84.76 79.96) (width 0.1524) (layer F.Cu) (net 46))
 (segment (start 71.81 89.71) (end 77.27 89.71) (width 0.1524) (layer F.Cu) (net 46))
 (segment (start 77.27 89.71) (end 84.76 82.22) (width 0.1524) (layer F.Cu) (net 46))
 (segment (start 82.22 82.22) (end 82.22 79.96) (width 0.1524) (layer F.Cu) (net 47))
 (segment (start 71.81 89.21) (end 75.23 89.21) (width 0.1524) (layer F.Cu) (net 47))
 (segment (start 75.23 89.21) (end 82.22 82.22) (width 0.1524) (layer F.Cu) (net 47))
 (segment (start 71.81 88.71) (end 74.46 88.71) (width 0.1524) (layer F.Cu) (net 48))
 (segment (start 79.68 83.49) (end 79.68 79.96) (width 0.1524) (layer F.Cu) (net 48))
 (segment (start 74.46 88.71) (end 79.68 83.49) (width 0.1524) (layer F.Cu) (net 48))
 (segment (start 77.14 84.76) (end 77.14 79.96) (width 0.1524) (layer F.Cu) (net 49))
 (segment (start 71.81 88.21) (end 73.69 88.21) (width 0.1524) (layer F.Cu) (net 49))
 (segment (start 73.69 88.21) (end 77.14 84.76) (width 0.1524) (layer F.Cu) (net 49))
 (segment (start 71.81 87.71) (end 72.92 87.71) (width 0.1524) (layer F.Cu) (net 50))
 (segment (start 74.6 86.03) (end 74.6 79.96) (width 0.1524) (layer F.Cu) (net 50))
 (segment (start 72.92 87.71) (end 74.6 86.03) (width 0.1524) (layer F.Cu) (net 50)))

